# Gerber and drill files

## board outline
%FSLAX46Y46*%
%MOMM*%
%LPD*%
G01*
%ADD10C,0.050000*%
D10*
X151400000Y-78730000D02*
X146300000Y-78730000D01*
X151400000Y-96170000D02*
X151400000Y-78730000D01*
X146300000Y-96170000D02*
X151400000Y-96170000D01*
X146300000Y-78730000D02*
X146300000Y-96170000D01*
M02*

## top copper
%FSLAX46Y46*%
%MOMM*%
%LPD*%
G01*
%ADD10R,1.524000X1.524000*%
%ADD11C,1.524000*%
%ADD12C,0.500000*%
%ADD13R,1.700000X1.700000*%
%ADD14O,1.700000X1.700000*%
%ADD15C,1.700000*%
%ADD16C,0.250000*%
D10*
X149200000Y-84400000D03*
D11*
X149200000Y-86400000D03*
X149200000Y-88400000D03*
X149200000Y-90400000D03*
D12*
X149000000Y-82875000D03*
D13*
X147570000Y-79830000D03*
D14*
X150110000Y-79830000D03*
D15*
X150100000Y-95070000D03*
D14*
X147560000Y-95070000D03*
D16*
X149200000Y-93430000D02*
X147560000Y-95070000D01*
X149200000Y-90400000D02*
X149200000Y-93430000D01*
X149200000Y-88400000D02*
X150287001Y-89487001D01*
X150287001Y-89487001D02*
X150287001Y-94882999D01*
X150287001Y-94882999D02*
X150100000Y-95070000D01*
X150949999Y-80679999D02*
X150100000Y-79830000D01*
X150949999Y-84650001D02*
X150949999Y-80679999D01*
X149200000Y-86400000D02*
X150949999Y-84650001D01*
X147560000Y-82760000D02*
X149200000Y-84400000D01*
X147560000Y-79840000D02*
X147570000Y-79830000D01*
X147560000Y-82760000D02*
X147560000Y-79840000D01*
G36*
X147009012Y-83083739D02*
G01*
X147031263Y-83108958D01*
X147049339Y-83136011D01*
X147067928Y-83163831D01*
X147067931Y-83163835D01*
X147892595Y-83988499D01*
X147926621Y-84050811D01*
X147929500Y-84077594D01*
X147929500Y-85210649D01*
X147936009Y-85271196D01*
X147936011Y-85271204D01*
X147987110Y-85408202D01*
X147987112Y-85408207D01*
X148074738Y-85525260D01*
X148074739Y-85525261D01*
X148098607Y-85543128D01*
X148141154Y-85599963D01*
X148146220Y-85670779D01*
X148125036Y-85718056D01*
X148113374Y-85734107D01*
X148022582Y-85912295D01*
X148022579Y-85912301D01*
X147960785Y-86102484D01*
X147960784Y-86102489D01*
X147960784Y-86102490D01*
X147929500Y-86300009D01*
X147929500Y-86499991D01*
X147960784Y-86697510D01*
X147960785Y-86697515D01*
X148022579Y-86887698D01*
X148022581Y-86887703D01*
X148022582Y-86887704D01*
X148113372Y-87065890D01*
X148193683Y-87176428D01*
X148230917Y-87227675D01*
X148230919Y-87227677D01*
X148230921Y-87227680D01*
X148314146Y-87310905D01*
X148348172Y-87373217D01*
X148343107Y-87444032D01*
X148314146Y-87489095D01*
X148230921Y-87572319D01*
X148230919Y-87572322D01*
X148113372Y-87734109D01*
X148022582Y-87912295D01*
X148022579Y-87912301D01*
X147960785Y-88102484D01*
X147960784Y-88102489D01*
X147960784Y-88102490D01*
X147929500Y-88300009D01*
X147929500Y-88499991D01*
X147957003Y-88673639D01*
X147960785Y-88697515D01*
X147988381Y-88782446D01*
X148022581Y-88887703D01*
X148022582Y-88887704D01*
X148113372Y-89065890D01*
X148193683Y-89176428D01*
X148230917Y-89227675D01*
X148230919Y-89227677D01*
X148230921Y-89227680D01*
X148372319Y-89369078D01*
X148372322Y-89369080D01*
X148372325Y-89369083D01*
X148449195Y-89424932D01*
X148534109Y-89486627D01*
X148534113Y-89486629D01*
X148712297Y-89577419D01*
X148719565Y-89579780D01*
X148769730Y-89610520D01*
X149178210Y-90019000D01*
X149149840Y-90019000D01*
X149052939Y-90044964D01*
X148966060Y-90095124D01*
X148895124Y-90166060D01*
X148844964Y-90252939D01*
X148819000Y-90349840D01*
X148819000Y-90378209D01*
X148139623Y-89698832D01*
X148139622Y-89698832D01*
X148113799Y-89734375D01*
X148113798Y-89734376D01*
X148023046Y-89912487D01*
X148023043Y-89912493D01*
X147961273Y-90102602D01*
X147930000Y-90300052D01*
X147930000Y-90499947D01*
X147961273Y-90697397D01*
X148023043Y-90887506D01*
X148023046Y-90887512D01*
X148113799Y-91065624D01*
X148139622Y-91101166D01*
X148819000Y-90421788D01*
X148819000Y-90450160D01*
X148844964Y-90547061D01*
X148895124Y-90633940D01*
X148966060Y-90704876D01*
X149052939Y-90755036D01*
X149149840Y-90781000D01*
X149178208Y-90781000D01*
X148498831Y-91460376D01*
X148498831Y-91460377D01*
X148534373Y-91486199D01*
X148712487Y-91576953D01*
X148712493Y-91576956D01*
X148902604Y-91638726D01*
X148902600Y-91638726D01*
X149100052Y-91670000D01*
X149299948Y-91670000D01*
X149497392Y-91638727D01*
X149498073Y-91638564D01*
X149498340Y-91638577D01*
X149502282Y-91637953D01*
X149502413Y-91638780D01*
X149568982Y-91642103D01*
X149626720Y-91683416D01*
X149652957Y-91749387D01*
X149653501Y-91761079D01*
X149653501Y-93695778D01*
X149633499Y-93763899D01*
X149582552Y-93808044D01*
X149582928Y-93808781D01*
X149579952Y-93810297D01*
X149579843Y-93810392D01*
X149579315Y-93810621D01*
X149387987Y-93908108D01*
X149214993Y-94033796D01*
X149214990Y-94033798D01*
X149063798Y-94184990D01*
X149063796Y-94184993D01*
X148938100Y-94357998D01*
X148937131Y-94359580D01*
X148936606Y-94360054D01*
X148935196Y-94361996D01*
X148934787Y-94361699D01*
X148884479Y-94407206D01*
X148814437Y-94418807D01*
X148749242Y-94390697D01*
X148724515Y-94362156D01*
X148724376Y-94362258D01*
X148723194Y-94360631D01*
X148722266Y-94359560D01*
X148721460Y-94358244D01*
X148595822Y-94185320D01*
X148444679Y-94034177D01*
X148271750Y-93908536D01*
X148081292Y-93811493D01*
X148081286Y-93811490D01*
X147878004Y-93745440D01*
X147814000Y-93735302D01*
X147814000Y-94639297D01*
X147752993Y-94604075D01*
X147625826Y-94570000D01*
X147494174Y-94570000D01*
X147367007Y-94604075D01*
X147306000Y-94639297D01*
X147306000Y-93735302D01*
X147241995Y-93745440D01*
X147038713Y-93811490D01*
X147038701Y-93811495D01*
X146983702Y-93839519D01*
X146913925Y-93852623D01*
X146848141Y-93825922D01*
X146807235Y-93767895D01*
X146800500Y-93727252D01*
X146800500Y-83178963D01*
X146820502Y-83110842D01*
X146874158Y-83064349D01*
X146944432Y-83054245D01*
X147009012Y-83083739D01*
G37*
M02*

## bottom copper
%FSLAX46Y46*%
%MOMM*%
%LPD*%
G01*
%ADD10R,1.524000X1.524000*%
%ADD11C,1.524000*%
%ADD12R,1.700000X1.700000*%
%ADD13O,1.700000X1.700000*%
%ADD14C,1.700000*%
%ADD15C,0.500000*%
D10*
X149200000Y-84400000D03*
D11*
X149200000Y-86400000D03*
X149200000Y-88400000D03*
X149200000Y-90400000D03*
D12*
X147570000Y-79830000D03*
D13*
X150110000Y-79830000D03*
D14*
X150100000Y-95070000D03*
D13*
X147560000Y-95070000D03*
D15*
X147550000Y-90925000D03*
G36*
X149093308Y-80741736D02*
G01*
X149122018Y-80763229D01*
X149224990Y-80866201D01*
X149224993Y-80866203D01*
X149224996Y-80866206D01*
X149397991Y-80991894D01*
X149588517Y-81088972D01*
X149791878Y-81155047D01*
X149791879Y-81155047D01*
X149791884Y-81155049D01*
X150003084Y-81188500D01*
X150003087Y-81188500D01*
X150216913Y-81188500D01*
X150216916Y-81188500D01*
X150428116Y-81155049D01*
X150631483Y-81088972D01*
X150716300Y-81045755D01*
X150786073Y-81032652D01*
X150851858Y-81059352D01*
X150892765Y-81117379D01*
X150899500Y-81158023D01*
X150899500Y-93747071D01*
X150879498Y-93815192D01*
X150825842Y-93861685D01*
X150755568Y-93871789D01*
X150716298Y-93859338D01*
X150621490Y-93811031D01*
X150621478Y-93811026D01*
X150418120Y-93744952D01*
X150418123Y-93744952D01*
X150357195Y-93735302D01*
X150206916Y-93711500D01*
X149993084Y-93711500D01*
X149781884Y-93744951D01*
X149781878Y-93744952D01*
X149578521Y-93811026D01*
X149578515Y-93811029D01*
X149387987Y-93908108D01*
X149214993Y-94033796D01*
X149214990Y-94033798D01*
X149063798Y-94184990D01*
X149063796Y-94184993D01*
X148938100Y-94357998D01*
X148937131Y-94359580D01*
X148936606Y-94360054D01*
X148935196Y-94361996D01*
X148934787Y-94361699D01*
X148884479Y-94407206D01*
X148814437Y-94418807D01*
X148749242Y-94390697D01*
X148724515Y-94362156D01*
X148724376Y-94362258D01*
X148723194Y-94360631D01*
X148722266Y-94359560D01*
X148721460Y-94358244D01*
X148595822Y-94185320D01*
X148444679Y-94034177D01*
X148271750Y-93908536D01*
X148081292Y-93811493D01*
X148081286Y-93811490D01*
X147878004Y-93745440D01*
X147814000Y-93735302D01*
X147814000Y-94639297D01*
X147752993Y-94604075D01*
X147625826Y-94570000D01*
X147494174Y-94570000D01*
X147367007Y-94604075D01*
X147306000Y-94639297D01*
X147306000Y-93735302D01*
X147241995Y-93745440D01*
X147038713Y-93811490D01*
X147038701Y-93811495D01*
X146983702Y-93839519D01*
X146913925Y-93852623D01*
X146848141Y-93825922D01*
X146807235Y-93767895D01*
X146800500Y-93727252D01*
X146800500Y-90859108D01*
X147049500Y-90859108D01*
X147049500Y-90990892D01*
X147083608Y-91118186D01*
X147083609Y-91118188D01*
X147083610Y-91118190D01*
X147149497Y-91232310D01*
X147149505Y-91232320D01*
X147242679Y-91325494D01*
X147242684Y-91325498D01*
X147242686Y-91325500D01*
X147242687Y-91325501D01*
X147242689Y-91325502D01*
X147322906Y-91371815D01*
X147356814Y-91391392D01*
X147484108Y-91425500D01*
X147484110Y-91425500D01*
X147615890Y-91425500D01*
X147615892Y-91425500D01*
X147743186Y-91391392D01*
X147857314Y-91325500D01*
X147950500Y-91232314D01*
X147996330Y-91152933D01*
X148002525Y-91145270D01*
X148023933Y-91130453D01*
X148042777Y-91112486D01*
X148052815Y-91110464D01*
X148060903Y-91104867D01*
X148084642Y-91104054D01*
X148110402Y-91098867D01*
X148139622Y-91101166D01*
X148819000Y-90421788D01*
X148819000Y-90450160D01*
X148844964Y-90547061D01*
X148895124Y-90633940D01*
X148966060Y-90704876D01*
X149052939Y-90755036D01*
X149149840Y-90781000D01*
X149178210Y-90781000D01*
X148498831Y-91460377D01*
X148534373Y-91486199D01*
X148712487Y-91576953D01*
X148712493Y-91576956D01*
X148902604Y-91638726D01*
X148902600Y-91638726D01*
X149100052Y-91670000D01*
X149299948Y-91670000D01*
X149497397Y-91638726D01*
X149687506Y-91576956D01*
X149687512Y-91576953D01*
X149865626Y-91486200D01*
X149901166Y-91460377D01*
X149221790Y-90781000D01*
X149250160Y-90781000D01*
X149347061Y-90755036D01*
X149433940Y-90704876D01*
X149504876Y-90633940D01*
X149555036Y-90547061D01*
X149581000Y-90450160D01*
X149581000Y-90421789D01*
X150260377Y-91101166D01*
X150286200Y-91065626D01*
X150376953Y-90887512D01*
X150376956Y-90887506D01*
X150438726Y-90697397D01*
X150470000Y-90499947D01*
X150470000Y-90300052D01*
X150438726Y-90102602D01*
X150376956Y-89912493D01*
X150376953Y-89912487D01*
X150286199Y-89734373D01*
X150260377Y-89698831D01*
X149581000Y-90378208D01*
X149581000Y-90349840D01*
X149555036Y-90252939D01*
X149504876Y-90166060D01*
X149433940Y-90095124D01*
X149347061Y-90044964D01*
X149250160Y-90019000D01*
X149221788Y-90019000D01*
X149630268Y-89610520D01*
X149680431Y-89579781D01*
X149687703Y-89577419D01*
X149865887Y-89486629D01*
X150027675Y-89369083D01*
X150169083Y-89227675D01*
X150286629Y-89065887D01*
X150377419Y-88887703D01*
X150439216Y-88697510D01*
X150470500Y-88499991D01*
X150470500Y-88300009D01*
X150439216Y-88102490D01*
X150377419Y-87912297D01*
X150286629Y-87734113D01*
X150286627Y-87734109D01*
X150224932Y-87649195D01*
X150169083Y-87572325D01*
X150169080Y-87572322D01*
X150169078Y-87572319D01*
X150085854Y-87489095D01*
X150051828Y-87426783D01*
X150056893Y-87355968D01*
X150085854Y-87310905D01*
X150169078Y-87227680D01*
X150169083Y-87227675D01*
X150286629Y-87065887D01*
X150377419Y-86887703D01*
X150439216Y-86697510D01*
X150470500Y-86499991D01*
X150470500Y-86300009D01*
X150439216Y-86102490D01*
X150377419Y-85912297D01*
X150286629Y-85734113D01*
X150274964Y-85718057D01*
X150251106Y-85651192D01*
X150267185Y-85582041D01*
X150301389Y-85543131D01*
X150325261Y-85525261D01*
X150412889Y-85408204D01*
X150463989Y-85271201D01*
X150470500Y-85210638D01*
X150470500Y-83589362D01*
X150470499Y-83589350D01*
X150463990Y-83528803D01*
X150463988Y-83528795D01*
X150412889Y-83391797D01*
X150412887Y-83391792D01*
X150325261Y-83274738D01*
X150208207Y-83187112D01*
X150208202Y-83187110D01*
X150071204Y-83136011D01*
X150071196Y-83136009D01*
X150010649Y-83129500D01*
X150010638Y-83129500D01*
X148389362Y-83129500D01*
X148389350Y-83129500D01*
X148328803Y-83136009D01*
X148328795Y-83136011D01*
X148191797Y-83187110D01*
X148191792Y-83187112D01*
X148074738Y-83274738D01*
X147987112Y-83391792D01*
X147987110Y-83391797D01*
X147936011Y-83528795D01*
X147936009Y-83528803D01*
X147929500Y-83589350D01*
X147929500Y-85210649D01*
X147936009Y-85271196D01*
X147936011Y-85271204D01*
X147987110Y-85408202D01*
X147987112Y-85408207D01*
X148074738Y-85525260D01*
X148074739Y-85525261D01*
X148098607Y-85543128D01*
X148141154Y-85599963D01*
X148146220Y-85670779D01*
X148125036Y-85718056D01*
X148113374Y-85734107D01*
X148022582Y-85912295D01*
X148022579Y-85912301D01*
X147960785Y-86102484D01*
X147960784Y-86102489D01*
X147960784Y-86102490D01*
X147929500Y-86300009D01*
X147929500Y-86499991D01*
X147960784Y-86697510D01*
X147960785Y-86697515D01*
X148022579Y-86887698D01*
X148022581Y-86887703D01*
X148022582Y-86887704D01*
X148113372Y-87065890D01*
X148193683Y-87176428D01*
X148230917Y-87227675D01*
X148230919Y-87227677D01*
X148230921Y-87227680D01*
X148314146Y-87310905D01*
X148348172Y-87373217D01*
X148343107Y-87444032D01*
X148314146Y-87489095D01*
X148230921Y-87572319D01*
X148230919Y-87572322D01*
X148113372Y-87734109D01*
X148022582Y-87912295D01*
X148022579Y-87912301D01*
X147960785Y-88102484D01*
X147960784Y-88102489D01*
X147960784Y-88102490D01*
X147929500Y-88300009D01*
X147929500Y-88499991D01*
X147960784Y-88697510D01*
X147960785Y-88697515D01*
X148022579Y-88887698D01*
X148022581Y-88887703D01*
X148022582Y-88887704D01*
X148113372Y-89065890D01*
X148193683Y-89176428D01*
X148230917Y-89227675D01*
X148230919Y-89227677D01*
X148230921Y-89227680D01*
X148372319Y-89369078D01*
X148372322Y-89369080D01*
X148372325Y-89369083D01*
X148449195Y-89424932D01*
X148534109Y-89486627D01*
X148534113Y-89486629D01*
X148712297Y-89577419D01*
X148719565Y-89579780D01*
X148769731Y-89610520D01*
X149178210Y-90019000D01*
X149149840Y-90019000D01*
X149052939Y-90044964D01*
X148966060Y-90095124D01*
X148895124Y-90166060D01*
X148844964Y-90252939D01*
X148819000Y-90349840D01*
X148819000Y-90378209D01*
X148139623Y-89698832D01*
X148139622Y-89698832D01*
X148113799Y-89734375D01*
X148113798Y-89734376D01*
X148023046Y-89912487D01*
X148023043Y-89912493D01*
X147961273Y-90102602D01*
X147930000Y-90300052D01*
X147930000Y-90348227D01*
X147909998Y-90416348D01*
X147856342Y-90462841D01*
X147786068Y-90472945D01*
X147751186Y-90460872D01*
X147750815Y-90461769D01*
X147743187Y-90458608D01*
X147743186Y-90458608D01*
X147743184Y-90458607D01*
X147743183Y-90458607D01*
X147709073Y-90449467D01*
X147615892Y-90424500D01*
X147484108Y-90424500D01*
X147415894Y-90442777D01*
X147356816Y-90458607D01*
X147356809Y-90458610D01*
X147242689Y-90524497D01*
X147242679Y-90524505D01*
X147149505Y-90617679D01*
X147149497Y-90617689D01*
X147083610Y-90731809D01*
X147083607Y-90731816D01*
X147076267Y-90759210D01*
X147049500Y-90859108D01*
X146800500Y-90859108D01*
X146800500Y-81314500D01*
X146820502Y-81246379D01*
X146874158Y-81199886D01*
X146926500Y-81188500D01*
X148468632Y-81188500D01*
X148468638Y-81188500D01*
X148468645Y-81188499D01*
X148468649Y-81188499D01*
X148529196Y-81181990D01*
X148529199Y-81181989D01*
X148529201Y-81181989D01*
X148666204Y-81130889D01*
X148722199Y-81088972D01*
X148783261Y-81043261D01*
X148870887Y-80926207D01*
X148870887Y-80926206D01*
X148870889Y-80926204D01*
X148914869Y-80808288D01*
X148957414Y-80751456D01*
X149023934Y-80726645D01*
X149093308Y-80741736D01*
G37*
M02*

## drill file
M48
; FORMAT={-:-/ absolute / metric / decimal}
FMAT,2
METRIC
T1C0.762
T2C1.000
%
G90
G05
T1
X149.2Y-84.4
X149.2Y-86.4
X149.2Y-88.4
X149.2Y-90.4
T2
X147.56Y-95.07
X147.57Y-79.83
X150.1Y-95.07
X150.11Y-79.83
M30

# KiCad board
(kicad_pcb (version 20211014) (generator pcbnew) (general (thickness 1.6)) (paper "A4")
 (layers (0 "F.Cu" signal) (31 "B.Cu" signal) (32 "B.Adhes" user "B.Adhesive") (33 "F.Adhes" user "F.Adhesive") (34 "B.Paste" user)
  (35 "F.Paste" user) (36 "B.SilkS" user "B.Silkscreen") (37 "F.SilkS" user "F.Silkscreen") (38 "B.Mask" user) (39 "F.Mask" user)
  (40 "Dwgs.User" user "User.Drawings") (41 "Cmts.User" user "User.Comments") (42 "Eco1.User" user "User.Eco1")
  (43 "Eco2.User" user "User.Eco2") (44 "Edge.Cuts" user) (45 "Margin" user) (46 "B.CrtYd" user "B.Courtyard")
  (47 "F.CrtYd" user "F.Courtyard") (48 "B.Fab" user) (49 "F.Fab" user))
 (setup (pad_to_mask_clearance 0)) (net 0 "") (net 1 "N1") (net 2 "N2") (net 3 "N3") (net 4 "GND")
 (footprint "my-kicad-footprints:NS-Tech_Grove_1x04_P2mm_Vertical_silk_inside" (layer "F.Cu") (at 149.2 84.4)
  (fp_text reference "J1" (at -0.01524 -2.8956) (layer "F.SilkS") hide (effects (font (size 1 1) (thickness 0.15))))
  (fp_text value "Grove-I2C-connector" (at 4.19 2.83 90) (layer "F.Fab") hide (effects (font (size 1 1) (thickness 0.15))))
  (pad "1" thru_hole rect locked (at 0 0) (size 1.524 1.524) (drill 0.762) (layers *.Cu *.Mask) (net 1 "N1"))
  (pad "2" thru_hole circle locked (at 0 2) (size 1.524 1.524) (drill 0.762) (layers *.Cu *.Mask) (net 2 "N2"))
  (pad "3" thru_hole circle locked (at 0 4) (size 1.524 1.524) (drill 0.762) (layers *.Cu *.Mask) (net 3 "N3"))
  (pad "4" thru_hole circle locked (at 0 6) (size 1.524 1.524) (drill 0.762) (layers *.Cu *.Mask) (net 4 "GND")))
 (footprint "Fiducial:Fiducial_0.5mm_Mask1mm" (layer "F.Cu") (at 149 82.875)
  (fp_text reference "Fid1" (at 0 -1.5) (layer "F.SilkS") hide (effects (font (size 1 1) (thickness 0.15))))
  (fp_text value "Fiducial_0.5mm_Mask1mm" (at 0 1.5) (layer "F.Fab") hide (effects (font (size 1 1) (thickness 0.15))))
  (pad "" smd circle locked (at 0 0) (size 0.5 0.5) (layers "F.Cu" "F.Mask") (solder_mask_margin 0.25) (clearance 0.25)))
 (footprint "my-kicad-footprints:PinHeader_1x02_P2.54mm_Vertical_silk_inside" (layer "B.Cu") (at 147.57 79.83 -90)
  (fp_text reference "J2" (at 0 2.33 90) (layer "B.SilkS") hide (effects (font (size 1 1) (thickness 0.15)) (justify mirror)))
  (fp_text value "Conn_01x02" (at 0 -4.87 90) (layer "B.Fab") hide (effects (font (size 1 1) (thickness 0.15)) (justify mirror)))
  (pad "1" thru_hole rect locked (at 0 0 270) (size 1.7 1.7) (drill 1) (layers *.Cu *.Mask) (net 1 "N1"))
  (pad "2" thru_hole oval locked (at 0 -2.54 270) (size 1.7 1.7) (drill 1) (layers *.Cu *.Mask) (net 2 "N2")))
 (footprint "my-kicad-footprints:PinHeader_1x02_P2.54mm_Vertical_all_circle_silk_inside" (layer "B.Cu") (at 150.1 95.07 90)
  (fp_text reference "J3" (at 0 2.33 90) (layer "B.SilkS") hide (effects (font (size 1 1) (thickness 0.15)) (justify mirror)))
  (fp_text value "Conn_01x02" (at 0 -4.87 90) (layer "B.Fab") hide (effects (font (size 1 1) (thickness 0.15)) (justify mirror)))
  (pad "1" thru_hole circle locked (at 0 0 90) (size 1.7 1.7) (drill 1) (layers *.Cu *.Mask) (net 3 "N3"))
  (pad "2" thru_hole oval locked (at 0 -2.54 90) (size 1.7 1.7) (drill 1) (layers *.Cu *.Mask) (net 4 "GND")))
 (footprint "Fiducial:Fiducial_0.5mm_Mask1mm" (layer "B.Cu") (at 147.55 90.925)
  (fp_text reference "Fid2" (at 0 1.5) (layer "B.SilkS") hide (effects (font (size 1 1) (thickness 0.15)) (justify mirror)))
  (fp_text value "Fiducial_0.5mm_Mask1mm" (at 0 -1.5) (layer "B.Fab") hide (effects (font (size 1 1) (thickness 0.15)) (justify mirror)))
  (pad "" smd circle locked (at 0 0) (size 0.5 0.5) (layers "B.Cu" "B.Mask") (solder_mask_margin 0.25) (clearance 0.25)))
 (gr_line (start 151.4 78.73) (end 146.3 78.73) (layer "Edge.Cuts") (width 0.05))
 (gr_line (start 151.4 96.17) (end 151.4 78.73) (layer "Edge.Cuts") (width 0.05))
 (gr_line (start 146.3 96.17) (end 151.4 96.17) (layer "Edge.Cuts") (width 0.05))
 (gr_line (start 146.3 78.73) (end 146.3 96.17) (layer "Edge.Cuts") (width 0.05))
 (segment (start 149.2 93.43) (end 147.56 95.07) (width 0.25) (layer "F.Cu") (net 4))
 (segment (start 149.2 90.4) (end 149.2 93.43) (width 0.25) (layer "F.Cu") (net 4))
 (segment (start 149.2 88.4) (end 150.287001 89.487001) (width 0.25) (layer "F.Cu") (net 3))
 (segment (start 150.287001 89.487001) (end 150.287001 94.882999) (width 0.25) (layer "F.Cu") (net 3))
 (segment (start 150.287001 94.882999) (end 150.1 95.07) (width 0.25) (layer "F.Cu") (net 3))
 (segment (start 150.949999 80.679999) (end 150.1 79.83) (width 0.25) (layer "F.Cu") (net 2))
 (segment (start 150.949999 84.650001) (end 150.949999 80.679999) (width 0.25) (layer "F.Cu") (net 2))
 (segment (start 149.2 86.4) (end 150.949999 84.650001) (width 0.25) (layer "F.Cu") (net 2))
 (segment (start 147.56 82.76) (end 149.2 84.4) (width 0.25) (layer "F.Cu") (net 1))
 (segment (start 147.56 79.84) (end 147.57 79.83) (width 0.25) (layer "F.Cu") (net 1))
 (segment (start 147.56 82.76) (end 147.56 79.84) (width 0.25) (layer "F.Cu") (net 1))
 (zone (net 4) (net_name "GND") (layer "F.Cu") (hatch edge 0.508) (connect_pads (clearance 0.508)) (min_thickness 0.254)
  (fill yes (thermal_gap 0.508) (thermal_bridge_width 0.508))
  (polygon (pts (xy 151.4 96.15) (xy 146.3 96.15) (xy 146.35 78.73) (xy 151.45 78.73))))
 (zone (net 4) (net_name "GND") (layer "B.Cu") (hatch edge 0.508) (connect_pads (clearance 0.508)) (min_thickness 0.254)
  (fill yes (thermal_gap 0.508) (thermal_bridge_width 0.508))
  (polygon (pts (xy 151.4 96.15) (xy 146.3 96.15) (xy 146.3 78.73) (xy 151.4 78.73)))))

